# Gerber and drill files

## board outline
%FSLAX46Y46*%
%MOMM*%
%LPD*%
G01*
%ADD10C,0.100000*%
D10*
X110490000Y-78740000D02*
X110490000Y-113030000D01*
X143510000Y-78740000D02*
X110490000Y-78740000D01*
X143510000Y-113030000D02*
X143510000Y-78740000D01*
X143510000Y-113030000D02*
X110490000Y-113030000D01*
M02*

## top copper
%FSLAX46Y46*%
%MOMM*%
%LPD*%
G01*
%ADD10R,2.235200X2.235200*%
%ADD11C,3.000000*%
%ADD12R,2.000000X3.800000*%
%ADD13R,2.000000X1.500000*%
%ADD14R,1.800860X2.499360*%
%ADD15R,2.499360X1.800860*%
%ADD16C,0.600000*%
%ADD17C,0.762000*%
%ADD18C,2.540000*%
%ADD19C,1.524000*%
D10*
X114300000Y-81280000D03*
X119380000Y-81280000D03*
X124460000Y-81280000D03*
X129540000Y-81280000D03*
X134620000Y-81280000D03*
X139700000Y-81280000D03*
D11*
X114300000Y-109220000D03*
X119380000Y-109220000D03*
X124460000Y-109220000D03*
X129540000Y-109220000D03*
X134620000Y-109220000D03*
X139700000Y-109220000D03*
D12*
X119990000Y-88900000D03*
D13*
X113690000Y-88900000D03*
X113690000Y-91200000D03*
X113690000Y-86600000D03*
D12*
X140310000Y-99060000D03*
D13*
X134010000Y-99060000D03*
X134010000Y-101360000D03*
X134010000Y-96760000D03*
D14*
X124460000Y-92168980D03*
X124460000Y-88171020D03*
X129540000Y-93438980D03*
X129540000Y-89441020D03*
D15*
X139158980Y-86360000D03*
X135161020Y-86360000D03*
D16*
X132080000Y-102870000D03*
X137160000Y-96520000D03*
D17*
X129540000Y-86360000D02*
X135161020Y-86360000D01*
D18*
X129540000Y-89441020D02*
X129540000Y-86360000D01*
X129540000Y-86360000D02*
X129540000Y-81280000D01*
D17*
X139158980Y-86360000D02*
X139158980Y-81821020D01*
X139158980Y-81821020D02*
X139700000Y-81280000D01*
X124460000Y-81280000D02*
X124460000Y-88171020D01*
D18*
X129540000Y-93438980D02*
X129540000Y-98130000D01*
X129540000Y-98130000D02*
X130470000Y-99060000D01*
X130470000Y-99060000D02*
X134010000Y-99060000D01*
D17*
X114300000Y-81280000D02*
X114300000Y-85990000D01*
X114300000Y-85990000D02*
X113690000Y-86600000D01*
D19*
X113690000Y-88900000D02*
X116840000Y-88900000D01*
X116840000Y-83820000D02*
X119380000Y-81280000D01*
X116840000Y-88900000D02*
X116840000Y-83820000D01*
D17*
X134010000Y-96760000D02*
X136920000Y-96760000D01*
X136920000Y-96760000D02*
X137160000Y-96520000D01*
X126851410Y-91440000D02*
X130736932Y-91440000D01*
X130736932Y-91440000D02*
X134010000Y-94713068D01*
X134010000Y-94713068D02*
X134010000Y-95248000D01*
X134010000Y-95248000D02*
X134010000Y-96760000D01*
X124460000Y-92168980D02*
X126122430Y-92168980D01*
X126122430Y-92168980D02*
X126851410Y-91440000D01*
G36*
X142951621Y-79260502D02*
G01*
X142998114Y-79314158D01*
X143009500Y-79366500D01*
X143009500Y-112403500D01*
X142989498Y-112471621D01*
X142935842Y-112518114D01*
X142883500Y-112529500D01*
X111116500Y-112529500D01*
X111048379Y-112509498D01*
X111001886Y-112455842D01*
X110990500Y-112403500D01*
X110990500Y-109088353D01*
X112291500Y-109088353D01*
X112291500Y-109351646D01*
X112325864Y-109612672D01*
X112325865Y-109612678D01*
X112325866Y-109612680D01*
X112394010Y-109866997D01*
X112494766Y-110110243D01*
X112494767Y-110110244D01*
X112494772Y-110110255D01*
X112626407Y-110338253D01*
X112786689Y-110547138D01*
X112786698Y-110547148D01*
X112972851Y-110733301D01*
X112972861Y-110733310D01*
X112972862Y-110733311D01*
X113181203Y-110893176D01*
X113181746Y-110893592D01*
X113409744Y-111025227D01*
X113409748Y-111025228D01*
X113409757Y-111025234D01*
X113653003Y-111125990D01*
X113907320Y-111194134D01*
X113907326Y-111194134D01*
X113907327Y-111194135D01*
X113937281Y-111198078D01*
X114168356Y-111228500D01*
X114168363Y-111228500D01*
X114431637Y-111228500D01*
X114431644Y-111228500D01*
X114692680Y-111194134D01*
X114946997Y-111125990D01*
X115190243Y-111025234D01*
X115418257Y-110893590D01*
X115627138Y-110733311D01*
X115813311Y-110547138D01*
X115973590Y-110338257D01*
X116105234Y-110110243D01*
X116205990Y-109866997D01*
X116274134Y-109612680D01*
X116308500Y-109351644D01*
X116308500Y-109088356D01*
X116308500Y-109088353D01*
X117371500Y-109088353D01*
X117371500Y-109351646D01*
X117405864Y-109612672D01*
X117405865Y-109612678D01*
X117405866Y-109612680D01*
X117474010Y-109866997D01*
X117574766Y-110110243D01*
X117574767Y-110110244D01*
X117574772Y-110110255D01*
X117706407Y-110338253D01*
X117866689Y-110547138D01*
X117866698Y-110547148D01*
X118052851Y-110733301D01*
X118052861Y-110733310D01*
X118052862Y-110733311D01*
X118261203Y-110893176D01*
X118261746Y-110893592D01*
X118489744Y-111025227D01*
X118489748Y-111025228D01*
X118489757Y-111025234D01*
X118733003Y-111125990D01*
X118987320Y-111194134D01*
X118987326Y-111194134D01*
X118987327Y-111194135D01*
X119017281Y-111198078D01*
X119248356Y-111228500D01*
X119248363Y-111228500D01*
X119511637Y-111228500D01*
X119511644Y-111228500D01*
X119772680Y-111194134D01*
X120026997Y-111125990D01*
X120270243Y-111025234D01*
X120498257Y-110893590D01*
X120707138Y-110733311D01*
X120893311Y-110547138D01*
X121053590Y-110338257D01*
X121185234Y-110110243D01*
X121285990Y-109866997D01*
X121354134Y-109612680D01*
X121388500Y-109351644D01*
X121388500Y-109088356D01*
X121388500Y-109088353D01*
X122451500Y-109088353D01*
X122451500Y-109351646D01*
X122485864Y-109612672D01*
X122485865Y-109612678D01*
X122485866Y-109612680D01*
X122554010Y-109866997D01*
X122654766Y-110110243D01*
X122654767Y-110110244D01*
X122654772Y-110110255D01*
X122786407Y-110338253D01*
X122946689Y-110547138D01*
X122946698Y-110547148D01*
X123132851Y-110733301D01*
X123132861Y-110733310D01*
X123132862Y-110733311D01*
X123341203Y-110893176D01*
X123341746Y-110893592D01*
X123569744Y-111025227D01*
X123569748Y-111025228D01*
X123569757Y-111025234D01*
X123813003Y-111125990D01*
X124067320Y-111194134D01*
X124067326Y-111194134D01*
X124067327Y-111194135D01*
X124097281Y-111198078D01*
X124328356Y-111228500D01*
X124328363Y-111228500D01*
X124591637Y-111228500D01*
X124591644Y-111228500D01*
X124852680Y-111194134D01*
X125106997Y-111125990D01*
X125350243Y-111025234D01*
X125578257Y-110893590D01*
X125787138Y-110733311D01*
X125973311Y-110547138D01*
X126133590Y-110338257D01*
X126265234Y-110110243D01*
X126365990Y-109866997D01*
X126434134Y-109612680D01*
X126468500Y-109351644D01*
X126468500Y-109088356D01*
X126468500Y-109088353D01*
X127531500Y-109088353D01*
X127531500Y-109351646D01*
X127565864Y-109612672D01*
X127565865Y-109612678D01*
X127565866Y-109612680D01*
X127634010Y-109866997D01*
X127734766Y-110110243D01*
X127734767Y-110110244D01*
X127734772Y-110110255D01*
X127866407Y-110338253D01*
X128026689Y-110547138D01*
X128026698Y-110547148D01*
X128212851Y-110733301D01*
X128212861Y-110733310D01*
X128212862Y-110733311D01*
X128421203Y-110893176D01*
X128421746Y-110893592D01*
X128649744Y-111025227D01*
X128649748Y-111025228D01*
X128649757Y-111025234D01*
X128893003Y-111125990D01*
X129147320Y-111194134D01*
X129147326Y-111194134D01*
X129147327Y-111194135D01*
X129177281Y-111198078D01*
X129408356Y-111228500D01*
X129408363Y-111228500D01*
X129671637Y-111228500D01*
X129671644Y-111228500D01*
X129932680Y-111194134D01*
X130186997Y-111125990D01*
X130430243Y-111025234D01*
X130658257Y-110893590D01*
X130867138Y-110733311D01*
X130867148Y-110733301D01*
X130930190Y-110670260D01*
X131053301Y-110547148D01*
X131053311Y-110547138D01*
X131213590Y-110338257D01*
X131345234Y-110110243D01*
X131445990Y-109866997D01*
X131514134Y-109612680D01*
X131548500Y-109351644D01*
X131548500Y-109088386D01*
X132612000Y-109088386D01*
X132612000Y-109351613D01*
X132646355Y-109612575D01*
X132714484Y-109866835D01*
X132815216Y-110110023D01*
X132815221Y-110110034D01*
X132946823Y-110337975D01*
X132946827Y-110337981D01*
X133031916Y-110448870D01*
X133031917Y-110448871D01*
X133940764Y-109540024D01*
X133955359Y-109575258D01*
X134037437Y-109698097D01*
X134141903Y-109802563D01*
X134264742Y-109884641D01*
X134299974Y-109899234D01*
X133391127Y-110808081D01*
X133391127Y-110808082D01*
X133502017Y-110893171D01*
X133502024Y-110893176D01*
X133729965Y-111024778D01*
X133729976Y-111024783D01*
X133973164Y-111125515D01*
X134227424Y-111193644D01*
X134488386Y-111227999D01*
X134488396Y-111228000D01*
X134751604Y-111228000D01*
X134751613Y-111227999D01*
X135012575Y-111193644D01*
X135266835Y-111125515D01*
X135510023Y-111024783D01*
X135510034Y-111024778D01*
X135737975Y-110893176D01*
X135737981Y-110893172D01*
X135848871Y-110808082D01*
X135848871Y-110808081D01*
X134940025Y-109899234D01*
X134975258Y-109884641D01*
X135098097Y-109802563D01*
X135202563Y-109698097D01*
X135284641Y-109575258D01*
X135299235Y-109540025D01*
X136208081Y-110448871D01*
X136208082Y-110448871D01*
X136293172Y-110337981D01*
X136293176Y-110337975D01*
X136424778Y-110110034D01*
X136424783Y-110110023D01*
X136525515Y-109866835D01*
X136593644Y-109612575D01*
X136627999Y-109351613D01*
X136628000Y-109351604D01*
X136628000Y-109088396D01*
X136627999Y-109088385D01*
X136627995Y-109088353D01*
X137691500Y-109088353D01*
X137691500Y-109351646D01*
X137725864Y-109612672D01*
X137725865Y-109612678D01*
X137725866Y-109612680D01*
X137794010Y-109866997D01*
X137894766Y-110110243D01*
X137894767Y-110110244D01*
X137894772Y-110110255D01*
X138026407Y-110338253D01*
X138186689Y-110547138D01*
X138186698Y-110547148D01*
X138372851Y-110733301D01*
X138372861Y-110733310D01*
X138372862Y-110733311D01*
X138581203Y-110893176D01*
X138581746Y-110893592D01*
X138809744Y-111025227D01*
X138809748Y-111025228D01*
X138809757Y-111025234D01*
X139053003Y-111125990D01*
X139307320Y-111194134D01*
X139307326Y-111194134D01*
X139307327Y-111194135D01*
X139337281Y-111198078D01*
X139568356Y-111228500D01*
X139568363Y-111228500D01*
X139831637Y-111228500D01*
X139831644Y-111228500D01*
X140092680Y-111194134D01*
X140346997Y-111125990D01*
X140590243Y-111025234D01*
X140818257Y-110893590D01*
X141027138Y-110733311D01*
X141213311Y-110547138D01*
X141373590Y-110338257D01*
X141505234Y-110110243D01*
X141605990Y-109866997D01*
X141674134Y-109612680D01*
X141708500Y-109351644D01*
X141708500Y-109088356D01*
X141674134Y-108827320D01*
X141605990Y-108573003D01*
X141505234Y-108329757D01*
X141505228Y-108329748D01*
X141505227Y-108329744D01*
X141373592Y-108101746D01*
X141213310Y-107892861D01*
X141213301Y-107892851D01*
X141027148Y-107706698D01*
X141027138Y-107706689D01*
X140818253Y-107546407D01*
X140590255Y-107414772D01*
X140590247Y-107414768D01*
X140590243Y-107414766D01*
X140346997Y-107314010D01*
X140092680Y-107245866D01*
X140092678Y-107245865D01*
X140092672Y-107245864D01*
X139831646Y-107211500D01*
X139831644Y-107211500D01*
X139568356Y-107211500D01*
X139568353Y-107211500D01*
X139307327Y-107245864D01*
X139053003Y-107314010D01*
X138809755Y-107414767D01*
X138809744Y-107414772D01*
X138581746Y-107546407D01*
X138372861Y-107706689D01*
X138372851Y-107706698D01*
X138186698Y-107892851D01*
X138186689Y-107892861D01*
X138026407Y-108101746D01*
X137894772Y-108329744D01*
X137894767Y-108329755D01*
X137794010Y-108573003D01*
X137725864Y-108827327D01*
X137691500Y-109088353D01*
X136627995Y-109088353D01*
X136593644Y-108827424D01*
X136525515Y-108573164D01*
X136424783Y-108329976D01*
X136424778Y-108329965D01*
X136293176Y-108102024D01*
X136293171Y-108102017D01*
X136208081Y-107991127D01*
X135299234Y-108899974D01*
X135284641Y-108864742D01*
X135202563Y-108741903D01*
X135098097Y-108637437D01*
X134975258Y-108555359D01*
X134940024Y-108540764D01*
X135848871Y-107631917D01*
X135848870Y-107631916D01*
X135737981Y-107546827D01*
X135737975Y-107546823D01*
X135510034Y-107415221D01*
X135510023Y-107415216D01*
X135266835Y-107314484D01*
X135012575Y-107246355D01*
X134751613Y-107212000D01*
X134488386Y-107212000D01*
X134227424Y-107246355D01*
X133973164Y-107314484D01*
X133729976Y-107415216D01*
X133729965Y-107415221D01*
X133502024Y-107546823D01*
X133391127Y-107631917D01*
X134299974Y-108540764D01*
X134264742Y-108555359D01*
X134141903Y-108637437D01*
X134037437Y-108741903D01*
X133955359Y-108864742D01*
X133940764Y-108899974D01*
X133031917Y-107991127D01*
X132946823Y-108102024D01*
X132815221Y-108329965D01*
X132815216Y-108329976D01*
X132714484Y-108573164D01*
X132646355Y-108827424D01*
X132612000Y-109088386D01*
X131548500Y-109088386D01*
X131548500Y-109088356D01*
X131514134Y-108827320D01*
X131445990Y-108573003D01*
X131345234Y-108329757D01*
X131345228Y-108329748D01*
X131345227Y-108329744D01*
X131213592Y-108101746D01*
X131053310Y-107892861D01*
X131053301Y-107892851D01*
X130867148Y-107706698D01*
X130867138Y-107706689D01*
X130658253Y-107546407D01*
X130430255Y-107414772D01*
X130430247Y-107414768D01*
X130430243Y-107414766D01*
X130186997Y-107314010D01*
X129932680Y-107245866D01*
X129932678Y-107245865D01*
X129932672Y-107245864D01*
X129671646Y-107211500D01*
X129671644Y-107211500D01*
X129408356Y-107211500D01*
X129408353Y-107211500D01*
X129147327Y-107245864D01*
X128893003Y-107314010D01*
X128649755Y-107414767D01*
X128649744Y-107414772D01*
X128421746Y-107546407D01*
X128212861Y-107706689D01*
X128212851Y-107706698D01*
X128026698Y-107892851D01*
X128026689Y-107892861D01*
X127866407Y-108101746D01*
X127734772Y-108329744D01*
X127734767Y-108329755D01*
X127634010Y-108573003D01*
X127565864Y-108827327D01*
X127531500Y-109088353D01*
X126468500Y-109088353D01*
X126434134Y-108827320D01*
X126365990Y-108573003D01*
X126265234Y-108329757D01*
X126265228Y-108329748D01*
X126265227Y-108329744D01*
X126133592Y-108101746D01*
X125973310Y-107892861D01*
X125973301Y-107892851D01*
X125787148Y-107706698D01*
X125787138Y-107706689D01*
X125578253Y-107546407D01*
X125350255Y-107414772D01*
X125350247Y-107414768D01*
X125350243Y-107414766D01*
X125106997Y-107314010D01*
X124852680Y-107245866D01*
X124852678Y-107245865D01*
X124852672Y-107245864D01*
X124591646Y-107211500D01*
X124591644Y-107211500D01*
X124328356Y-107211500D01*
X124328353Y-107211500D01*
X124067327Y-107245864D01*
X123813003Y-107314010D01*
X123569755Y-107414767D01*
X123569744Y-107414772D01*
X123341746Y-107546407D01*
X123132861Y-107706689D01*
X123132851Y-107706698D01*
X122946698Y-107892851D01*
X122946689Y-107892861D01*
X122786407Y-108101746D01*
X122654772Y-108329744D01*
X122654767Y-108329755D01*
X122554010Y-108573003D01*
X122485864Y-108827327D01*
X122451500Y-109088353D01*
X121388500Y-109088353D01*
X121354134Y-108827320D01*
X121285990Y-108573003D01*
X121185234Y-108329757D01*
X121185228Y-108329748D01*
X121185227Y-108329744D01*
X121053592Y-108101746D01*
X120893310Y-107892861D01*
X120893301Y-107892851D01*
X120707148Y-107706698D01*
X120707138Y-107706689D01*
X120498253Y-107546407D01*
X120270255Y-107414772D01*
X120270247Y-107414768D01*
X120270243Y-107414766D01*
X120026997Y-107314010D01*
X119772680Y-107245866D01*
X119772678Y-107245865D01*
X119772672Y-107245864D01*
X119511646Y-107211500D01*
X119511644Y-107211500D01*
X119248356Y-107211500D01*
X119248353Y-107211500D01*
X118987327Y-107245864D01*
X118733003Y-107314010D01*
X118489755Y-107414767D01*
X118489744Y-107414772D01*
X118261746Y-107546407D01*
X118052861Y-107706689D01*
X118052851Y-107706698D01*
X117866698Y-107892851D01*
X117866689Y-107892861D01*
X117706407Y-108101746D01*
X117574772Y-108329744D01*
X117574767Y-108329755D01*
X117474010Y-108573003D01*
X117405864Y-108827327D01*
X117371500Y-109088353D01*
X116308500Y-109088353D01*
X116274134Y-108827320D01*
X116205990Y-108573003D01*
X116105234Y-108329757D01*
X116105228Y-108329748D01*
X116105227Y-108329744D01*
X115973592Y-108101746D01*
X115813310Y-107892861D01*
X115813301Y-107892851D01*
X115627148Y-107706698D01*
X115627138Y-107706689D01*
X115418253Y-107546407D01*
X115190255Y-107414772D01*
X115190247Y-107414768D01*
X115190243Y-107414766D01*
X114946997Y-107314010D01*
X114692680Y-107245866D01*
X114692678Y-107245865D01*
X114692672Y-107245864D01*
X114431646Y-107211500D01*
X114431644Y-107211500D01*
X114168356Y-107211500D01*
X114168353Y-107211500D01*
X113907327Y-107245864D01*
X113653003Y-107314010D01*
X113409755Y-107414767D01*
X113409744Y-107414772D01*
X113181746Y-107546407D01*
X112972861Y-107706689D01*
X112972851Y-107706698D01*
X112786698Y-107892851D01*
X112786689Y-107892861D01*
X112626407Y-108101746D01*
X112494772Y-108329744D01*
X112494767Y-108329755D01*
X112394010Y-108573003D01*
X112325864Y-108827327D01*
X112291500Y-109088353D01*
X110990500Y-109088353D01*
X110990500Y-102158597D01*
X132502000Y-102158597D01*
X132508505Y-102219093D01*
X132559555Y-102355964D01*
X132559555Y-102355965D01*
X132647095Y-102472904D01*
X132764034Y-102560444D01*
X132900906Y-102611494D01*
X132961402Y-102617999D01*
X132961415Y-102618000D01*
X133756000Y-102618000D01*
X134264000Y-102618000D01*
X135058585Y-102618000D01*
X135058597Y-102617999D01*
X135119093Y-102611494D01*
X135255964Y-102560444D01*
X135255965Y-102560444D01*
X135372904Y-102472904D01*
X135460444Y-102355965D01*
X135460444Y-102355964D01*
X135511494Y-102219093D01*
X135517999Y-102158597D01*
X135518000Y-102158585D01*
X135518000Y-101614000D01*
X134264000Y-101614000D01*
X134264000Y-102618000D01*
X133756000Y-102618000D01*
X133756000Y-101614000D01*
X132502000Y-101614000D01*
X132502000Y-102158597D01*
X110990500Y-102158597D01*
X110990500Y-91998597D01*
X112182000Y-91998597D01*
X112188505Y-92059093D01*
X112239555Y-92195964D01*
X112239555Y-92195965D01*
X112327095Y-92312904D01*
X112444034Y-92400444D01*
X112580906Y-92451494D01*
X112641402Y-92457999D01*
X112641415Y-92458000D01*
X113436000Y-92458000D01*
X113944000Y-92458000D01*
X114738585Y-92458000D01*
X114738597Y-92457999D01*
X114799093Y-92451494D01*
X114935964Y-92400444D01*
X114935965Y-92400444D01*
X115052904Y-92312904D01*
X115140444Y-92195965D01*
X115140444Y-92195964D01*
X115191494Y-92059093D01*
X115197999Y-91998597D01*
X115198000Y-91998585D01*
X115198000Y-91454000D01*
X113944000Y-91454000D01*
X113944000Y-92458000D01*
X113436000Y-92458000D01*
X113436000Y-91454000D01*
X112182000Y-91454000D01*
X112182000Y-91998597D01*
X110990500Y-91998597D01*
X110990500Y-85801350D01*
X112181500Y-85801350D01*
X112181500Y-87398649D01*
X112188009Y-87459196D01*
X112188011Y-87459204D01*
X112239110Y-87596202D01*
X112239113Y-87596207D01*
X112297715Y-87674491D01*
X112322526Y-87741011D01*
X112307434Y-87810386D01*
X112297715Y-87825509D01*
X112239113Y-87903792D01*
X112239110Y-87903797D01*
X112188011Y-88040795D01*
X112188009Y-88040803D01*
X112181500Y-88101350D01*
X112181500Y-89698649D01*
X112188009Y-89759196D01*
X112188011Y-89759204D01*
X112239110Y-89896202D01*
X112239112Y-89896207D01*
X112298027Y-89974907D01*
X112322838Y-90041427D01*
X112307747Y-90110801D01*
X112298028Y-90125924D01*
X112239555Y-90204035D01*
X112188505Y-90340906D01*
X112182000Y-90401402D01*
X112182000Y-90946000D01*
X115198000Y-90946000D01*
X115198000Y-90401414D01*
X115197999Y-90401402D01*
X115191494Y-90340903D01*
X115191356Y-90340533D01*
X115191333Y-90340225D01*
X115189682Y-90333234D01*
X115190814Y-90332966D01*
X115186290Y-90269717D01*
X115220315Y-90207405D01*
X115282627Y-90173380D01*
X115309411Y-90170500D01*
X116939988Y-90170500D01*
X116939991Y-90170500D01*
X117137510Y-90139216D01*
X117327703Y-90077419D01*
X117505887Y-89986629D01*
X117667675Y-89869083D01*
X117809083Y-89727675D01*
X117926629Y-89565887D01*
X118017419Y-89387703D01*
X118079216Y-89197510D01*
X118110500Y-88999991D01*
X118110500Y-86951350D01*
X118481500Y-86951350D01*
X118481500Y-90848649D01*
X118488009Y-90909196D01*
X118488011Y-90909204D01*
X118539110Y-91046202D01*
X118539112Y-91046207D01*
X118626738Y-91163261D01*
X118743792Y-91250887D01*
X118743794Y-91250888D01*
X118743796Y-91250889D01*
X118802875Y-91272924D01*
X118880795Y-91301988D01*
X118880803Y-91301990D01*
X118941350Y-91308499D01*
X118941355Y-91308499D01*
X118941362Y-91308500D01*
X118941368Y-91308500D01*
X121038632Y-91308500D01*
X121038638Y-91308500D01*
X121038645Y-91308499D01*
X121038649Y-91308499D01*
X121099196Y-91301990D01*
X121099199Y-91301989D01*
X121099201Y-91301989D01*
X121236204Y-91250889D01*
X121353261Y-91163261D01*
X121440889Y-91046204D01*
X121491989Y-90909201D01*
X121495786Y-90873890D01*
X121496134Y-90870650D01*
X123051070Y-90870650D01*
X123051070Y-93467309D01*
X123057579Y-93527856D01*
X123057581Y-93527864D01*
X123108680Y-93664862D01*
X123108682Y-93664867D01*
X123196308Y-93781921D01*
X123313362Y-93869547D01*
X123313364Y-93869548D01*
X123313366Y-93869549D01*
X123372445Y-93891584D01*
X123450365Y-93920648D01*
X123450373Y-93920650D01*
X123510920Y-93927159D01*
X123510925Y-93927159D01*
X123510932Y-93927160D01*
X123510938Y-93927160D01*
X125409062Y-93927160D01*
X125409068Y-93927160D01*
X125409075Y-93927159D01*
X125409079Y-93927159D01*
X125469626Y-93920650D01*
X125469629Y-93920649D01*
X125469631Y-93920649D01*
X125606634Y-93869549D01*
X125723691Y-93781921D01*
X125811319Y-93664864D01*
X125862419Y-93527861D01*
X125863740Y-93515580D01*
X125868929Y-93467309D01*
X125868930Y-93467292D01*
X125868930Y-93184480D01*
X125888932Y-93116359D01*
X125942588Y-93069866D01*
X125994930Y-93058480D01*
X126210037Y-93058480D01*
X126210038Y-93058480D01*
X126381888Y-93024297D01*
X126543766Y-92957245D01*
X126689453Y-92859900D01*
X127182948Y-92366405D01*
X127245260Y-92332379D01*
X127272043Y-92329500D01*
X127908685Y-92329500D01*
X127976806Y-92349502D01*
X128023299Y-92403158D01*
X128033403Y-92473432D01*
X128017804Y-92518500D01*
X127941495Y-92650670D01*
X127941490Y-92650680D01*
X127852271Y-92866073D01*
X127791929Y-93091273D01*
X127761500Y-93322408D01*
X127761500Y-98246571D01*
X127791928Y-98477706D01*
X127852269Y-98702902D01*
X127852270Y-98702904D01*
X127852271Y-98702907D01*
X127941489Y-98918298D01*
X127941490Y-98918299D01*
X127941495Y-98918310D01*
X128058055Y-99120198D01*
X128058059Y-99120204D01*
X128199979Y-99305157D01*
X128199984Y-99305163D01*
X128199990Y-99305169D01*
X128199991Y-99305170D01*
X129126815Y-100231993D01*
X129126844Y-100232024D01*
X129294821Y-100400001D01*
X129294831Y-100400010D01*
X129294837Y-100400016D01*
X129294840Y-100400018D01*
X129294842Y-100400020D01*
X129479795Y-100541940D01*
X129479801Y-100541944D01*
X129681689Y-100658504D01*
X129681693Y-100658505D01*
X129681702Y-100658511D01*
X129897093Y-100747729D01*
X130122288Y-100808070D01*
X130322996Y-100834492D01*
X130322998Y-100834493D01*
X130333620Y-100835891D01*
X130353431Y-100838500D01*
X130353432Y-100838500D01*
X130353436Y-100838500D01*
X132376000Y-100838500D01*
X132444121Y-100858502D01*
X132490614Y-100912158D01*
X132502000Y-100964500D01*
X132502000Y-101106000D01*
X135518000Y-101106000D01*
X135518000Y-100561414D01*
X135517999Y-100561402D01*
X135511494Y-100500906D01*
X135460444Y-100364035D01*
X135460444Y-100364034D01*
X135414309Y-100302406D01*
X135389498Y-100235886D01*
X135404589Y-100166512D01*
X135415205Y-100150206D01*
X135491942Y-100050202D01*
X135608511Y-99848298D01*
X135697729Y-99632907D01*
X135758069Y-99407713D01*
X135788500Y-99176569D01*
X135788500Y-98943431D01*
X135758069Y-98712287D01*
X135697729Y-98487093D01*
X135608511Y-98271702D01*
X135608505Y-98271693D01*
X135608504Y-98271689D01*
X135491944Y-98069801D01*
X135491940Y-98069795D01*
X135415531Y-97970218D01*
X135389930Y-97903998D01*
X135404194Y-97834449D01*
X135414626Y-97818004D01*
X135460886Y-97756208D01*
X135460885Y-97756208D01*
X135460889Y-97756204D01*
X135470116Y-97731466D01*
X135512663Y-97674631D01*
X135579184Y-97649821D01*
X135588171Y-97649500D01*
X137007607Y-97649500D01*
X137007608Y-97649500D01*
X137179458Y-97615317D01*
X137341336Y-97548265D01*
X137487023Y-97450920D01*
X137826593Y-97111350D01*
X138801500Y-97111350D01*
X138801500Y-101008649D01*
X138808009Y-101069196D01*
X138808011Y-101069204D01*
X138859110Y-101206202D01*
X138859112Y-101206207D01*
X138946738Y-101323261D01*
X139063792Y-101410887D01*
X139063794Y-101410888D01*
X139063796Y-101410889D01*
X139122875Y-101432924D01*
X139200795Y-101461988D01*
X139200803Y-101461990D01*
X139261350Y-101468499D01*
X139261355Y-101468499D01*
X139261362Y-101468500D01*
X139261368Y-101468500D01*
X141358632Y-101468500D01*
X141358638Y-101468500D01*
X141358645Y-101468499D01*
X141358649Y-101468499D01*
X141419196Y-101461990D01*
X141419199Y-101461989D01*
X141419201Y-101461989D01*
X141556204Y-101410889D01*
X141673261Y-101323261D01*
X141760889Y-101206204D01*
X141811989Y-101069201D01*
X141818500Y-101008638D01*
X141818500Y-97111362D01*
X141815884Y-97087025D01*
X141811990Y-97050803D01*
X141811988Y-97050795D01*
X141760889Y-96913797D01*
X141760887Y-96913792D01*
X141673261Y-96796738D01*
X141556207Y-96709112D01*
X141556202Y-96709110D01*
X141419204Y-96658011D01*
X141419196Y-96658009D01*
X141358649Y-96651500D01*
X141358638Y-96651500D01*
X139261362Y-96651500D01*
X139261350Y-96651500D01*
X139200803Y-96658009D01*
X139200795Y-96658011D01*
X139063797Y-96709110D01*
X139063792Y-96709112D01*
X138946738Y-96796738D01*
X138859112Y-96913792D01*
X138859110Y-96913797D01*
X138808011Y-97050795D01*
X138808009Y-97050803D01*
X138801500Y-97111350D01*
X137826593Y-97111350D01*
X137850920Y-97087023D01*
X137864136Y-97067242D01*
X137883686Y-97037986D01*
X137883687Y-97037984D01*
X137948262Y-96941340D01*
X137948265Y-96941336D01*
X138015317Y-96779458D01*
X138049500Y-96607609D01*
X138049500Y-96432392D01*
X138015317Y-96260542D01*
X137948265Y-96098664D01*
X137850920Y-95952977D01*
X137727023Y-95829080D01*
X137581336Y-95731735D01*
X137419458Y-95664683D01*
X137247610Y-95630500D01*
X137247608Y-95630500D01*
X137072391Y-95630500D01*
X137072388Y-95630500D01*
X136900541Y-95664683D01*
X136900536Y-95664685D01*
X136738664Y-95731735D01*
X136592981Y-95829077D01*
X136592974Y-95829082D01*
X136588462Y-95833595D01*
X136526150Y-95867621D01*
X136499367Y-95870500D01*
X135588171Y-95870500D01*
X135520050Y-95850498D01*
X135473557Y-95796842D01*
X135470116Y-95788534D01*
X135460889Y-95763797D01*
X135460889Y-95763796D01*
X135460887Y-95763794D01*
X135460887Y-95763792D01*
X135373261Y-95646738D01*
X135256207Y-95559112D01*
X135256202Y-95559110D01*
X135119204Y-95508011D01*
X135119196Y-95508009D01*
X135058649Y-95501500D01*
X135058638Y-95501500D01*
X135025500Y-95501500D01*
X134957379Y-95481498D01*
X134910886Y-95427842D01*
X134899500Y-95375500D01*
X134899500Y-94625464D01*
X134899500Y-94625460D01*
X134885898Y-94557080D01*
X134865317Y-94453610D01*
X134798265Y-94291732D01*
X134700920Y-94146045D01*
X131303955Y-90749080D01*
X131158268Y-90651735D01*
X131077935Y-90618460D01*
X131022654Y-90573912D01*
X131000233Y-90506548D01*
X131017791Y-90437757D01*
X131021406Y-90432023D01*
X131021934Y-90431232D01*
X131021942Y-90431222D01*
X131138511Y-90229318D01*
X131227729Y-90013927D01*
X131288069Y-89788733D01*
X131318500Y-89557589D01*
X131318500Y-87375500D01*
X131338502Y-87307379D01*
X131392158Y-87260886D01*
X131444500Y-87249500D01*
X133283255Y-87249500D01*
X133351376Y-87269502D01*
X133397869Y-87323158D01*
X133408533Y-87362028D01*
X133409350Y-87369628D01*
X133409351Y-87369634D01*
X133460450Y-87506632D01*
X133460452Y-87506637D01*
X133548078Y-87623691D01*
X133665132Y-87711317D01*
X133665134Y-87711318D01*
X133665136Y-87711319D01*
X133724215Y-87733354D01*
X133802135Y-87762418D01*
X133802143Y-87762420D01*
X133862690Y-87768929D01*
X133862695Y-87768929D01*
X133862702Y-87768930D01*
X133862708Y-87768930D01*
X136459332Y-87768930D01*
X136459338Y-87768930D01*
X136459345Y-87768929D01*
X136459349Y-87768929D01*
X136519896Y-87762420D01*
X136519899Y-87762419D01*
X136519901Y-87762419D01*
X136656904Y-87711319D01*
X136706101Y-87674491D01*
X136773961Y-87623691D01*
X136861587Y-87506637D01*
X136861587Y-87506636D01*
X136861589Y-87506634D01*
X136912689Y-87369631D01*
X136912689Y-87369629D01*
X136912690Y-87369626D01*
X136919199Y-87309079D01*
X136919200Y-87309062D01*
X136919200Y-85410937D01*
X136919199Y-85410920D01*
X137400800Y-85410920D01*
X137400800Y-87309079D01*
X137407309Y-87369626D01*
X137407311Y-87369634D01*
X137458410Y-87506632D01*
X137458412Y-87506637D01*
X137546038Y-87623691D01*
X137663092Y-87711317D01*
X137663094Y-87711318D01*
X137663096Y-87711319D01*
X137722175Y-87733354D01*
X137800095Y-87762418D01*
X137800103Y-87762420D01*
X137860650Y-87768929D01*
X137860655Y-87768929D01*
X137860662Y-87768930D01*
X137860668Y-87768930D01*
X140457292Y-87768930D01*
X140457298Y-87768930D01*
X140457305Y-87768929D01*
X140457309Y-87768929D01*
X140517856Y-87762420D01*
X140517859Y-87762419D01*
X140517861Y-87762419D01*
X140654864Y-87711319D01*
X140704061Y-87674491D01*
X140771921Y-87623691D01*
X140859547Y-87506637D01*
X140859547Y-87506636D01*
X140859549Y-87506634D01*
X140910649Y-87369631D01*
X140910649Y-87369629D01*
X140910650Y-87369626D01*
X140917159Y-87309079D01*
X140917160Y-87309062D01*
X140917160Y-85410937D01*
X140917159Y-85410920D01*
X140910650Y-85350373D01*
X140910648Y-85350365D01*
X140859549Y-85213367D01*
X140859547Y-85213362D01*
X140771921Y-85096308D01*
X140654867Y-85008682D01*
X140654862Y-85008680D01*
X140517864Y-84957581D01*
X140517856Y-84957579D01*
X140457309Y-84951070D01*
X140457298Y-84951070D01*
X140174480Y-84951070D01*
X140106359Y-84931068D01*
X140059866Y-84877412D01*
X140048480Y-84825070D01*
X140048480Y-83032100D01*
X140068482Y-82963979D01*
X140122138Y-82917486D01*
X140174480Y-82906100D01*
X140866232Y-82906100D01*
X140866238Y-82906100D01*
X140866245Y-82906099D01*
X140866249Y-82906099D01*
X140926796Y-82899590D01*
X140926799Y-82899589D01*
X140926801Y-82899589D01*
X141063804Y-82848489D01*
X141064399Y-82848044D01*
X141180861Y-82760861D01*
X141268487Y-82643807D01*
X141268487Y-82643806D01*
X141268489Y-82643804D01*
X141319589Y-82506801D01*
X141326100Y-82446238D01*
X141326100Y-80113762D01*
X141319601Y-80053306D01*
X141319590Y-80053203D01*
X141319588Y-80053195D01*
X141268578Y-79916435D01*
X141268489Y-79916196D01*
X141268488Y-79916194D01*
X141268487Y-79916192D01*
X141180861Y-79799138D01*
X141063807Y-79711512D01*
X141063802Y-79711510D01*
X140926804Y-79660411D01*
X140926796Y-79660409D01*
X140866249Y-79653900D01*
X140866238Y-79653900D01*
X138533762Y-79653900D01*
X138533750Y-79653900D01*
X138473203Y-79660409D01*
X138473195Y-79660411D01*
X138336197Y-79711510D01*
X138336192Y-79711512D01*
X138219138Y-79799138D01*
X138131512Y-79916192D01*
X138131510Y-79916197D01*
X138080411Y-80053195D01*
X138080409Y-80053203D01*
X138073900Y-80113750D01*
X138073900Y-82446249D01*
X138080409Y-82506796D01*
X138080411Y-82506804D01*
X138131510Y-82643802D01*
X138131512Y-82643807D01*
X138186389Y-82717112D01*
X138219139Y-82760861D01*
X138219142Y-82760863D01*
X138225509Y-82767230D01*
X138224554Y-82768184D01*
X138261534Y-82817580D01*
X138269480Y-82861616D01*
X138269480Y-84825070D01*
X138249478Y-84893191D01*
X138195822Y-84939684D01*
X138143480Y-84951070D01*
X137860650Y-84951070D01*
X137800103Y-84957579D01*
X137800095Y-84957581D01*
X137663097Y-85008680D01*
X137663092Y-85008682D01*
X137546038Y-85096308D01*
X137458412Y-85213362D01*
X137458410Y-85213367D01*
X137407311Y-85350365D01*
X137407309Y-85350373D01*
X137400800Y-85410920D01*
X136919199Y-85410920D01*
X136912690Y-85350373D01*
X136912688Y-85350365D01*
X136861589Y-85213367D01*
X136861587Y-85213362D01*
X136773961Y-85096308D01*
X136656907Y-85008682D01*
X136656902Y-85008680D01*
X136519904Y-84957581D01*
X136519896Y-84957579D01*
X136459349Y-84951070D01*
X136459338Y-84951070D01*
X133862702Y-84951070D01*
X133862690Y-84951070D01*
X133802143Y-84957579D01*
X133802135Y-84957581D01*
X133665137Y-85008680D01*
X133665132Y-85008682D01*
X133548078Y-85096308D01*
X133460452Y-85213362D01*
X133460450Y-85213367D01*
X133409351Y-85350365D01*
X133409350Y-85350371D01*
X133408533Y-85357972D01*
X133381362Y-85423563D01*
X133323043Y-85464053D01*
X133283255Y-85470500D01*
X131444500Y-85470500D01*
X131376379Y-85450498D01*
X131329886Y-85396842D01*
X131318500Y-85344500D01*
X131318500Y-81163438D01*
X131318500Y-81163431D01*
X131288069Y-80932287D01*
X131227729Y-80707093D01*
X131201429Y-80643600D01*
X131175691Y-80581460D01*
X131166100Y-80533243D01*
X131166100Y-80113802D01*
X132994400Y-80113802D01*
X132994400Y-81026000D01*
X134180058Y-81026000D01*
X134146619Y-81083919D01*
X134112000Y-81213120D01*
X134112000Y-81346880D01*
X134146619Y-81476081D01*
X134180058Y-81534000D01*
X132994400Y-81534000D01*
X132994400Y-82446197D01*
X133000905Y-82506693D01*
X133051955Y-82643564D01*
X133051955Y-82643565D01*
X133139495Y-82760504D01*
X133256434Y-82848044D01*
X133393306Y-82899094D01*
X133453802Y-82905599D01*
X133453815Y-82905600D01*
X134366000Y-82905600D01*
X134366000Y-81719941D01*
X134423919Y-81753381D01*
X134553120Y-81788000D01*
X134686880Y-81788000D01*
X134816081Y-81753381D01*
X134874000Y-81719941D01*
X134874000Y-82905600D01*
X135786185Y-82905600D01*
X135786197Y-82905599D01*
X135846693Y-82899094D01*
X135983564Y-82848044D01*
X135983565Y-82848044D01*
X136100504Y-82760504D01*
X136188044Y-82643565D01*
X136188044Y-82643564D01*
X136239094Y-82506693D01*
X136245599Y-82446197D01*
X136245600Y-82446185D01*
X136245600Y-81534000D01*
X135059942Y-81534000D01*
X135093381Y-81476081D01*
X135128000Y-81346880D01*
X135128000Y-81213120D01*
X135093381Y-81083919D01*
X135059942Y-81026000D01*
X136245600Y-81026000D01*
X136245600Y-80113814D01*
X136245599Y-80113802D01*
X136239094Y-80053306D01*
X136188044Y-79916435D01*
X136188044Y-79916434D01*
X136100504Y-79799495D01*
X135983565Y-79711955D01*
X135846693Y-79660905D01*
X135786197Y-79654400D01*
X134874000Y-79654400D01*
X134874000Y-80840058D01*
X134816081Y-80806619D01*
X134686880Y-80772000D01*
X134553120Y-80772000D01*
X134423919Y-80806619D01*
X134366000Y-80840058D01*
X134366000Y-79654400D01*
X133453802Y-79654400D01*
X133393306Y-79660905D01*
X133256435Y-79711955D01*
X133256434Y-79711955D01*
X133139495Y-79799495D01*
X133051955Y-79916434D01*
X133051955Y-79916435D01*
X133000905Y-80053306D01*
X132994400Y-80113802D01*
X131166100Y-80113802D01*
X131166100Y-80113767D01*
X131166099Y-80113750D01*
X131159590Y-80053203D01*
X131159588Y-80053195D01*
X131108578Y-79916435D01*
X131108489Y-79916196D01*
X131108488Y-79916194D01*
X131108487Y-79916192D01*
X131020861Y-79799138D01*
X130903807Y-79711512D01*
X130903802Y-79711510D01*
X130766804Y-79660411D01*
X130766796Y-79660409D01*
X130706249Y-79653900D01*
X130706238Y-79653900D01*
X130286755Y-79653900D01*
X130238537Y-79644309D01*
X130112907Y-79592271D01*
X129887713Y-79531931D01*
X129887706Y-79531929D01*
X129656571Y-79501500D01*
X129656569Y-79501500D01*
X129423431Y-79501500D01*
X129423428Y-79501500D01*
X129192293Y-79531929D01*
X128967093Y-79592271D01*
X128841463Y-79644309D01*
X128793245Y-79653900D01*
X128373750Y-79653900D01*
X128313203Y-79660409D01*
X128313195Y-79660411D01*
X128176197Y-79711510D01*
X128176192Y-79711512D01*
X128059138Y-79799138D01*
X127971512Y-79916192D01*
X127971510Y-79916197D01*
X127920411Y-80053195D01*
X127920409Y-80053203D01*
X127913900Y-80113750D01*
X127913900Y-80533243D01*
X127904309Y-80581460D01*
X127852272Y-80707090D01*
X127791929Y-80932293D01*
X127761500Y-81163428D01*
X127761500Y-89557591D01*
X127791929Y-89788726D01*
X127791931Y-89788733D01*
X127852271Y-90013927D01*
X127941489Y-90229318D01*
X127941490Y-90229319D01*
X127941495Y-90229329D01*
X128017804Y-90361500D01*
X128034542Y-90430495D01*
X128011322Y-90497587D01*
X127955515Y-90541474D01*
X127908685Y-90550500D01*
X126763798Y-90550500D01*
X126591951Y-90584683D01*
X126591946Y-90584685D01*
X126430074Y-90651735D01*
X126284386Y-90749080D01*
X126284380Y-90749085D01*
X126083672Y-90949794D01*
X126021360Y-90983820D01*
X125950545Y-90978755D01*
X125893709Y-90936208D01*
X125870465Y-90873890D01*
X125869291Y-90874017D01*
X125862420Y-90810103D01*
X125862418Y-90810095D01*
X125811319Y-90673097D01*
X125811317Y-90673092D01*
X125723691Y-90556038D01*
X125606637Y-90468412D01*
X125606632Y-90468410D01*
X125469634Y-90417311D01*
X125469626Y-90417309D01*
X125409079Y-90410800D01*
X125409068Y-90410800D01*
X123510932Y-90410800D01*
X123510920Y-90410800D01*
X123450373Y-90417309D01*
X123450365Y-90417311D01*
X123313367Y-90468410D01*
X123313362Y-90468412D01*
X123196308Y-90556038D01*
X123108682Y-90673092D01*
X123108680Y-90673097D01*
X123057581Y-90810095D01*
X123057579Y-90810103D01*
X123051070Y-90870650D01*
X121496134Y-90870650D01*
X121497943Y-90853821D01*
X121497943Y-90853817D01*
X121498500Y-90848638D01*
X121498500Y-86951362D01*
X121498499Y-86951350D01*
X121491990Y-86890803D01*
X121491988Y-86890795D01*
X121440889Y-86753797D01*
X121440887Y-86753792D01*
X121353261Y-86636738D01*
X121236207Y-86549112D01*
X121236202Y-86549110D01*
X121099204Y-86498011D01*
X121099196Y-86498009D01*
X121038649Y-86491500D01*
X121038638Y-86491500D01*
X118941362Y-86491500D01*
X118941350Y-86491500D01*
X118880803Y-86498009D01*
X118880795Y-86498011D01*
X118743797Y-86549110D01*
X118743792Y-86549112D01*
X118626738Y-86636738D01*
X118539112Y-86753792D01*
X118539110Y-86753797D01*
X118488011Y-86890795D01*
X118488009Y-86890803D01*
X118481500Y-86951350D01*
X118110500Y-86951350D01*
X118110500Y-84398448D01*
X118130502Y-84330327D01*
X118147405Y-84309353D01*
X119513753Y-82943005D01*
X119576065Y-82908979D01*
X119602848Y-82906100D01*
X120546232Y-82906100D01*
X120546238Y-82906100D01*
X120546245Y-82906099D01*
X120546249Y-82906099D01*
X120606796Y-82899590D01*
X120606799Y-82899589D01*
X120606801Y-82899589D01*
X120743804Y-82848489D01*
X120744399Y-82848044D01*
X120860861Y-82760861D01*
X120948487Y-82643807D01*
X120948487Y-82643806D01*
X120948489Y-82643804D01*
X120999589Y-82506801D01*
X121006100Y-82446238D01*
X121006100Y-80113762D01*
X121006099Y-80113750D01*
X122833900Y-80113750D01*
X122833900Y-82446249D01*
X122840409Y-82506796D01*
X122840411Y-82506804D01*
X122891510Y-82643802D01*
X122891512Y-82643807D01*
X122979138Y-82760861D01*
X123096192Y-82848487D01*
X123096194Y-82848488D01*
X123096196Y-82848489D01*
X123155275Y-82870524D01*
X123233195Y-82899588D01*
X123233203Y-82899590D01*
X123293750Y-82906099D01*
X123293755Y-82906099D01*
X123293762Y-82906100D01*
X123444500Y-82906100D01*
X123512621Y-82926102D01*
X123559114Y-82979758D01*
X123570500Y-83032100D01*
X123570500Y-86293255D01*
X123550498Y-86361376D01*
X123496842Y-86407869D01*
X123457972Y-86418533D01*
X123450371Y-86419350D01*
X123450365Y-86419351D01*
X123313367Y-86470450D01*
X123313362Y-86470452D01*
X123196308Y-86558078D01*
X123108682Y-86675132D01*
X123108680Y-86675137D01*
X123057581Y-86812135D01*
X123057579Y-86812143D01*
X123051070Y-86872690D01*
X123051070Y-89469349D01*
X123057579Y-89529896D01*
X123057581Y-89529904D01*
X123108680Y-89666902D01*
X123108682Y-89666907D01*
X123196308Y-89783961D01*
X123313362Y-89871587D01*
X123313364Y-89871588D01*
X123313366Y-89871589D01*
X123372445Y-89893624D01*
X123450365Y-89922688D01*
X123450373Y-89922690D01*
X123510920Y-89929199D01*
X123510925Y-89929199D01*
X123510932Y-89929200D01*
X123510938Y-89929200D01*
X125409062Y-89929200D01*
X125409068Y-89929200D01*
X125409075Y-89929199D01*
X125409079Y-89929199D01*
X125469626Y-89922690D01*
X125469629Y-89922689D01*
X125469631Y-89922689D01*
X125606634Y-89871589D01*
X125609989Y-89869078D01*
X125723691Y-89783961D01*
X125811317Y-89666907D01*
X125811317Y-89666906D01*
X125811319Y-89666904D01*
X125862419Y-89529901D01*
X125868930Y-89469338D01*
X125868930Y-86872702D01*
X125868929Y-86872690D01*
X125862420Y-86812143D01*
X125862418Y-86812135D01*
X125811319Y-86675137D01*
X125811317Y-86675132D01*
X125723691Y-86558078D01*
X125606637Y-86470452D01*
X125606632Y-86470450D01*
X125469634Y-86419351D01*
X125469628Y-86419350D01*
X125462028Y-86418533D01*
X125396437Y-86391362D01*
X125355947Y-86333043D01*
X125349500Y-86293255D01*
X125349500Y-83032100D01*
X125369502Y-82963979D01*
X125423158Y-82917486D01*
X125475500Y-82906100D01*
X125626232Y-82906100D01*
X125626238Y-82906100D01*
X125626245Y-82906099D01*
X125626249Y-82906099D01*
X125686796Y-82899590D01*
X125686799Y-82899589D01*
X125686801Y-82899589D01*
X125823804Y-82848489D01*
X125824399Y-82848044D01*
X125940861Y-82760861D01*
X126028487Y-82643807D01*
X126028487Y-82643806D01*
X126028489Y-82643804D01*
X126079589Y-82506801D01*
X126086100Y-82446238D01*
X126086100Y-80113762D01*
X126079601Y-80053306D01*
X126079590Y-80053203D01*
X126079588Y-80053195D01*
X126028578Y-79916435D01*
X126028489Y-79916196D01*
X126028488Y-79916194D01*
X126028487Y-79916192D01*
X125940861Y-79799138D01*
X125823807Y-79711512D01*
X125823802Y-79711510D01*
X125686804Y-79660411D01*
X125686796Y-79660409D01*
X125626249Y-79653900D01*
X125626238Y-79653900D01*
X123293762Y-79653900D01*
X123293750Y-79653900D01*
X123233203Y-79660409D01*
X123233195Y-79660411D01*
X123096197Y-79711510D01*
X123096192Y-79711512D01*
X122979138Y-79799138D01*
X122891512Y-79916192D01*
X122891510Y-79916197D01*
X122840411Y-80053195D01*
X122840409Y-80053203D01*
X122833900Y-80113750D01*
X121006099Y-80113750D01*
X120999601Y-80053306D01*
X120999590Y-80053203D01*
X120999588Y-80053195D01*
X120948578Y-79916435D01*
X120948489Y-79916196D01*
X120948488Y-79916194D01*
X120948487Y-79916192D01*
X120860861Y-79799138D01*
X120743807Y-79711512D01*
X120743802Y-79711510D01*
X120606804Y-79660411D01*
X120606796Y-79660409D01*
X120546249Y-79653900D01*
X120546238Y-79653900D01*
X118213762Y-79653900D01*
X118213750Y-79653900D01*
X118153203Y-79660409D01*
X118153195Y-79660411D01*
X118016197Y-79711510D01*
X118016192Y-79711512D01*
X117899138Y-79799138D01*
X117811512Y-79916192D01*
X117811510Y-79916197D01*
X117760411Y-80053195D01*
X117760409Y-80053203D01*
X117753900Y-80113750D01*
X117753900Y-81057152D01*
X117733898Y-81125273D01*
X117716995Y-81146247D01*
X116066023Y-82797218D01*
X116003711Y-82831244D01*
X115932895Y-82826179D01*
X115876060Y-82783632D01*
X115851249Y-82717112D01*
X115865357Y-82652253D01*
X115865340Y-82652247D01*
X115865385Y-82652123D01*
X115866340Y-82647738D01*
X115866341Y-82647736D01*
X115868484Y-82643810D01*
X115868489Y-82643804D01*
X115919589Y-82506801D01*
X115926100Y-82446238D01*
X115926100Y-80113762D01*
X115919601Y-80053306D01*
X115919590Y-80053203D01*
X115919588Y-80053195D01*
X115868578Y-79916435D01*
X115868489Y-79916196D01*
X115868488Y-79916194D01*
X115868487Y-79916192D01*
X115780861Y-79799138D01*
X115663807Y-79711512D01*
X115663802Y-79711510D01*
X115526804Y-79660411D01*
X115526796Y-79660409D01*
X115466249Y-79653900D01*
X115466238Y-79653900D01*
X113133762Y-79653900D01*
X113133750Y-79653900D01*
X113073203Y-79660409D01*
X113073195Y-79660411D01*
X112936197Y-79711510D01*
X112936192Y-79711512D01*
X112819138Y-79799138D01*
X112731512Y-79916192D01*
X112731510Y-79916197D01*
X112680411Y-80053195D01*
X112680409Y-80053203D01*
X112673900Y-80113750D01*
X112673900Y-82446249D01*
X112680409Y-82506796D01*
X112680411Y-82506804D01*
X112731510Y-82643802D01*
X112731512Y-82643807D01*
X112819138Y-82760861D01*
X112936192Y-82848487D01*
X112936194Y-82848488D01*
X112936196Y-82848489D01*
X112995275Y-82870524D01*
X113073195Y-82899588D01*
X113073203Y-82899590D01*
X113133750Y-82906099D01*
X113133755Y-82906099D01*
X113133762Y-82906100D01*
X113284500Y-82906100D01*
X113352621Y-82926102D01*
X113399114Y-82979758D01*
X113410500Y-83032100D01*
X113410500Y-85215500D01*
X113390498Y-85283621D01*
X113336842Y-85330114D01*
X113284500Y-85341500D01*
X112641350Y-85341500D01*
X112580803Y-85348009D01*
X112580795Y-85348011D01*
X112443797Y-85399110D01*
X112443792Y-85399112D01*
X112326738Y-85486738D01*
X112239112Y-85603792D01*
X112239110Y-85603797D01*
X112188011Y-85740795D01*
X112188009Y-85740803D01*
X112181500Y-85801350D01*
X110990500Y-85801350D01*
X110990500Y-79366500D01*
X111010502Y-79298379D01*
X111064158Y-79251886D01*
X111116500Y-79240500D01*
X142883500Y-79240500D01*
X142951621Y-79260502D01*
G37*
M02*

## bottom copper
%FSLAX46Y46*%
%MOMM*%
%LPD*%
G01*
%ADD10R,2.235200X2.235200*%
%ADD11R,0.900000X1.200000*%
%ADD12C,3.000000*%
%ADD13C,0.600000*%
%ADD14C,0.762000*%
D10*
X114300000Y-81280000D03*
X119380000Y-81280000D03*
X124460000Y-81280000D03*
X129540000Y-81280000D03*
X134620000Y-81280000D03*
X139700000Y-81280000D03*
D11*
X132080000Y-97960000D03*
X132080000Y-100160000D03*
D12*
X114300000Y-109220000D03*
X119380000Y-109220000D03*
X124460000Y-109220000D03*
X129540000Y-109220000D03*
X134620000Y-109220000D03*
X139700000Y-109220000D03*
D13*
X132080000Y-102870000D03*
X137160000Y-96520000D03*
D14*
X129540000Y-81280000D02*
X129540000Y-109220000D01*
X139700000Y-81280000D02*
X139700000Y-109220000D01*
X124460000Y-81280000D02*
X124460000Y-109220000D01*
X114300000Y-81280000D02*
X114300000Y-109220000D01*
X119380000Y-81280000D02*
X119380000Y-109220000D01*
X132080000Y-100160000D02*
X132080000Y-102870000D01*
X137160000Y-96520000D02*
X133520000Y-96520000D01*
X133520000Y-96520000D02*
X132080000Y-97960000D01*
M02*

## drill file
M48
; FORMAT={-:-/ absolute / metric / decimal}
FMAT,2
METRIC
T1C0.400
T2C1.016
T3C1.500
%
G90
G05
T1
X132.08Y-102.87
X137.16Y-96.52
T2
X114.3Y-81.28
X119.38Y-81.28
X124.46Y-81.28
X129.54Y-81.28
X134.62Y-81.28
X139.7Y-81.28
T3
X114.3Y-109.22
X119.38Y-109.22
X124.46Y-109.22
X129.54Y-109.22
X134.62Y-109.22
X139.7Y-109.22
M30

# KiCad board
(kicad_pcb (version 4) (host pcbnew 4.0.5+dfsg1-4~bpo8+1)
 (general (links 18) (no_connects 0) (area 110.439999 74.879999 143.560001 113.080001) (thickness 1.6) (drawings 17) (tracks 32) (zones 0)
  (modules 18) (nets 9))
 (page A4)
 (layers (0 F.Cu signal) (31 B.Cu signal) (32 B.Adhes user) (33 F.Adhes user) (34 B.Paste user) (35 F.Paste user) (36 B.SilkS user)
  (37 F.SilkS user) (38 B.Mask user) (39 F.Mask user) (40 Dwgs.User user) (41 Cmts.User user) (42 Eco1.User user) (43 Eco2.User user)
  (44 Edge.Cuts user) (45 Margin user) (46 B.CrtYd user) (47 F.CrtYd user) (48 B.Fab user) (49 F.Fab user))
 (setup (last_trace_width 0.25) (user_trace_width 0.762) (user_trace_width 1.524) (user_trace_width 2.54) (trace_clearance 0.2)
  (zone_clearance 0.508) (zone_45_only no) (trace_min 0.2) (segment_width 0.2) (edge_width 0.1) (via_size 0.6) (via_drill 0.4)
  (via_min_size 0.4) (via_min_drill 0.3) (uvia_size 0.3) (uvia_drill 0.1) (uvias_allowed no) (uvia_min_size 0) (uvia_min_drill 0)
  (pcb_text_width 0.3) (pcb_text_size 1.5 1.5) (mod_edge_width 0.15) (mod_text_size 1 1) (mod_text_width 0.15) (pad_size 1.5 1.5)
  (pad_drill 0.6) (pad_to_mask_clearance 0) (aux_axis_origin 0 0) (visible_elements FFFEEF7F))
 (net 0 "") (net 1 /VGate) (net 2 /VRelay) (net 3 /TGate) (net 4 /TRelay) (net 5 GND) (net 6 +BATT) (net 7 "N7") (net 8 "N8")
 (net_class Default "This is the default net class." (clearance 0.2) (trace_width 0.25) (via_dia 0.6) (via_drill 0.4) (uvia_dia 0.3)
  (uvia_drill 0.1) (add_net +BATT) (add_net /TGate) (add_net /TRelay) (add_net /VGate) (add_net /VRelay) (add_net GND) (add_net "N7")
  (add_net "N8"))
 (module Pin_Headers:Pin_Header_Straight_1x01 (layer B.Cu) (at 114.3 81.28)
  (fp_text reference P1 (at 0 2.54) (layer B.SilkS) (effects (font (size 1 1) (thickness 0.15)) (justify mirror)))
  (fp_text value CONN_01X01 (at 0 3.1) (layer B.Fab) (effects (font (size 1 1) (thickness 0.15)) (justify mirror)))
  (pad 1 thru_hole rect (at 0 0) (size 2.2352 2.2352) (drill 1.016) (layers *.Cu *.Mask) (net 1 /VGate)))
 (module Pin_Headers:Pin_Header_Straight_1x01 (layer B.Cu) (at 119.38 81.28)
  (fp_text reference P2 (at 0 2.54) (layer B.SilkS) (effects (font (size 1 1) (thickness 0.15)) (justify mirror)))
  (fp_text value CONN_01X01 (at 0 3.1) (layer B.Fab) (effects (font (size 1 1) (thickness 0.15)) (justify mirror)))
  (pad 1 thru_hole rect (at 0 0) (size 2.2352 2.2352) (drill 1.016) (layers *.Cu *.Mask) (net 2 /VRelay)))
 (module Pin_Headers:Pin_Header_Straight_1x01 (layer B.Cu) (at 124.46 81.28)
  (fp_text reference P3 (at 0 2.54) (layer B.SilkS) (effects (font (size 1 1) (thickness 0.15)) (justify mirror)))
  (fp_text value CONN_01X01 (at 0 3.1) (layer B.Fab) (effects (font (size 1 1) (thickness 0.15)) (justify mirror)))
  (pad 1 thru_hole rect (at 0 0) (size 2.2352 2.2352) (drill 1.016) (layers *.Cu *.Mask) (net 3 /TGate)))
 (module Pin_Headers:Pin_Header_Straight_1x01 (layer B.Cu) (at 129.54 81.28)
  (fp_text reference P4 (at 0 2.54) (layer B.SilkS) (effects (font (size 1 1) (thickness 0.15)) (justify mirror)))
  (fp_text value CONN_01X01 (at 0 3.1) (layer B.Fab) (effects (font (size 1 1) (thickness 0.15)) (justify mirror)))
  (pad 1 thru_hole rect (at 0 0) (size 2.2352 2.2352) (drill 1.016) (layers *.Cu *.Mask) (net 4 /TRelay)))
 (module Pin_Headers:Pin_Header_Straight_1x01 (layer B.Cu) (at 134.62 81.28)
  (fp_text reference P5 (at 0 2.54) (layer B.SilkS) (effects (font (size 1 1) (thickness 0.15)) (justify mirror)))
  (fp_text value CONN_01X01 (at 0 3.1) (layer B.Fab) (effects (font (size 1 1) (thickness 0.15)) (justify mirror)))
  (pad 1 thru_hole rect (at 0 0) (size 2.2352 2.2352) (drill 1.016) (layers *.Cu *.Mask) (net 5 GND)))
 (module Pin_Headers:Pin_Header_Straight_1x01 (layer B.Cu) (at 139.7 81.28)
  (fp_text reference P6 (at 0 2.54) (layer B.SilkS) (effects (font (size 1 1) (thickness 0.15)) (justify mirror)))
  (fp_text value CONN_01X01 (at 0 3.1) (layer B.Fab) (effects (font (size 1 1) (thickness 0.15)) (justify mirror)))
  (pad 1 thru_hole rect (at 0 0) (size 2.2352 2.2352) (drill 1.016) (layers *.Cu *.Mask) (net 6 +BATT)))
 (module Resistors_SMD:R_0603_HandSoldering (layer B.Cu) (at 132.08 99.06 270)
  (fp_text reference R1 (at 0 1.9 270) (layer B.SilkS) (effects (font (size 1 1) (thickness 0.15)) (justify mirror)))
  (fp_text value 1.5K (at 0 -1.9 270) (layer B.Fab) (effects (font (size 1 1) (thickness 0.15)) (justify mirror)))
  (pad 1 smd rect (at -1.1 0 270) (size 1.2 0.9) (layers B.Cu B.Paste B.Mask) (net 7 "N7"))
  (pad 2 smd rect (at 1.1 0 270) (size 1.2 0.9) (layers B.Cu B.Paste B.Mask) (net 5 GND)))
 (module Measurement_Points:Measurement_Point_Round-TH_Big (layer B.Cu) (at 114.3 109.22)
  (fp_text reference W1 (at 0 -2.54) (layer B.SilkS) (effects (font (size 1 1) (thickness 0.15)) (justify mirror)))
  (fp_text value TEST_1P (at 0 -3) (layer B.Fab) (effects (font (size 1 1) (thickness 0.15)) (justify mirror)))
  (pad 1 thru_hole circle (at 0 0) (size 3 3) (drill 1.5) (layers *.Cu *.Mask) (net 1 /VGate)))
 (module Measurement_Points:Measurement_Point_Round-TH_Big (layer B.Cu) (at 119.38 109.22)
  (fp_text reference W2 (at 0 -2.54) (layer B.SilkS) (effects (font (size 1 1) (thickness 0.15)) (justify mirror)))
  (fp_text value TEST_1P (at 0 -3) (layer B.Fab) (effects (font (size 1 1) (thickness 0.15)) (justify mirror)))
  (pad 1 thru_hole circle (at 0 0) (size 3 3) (drill 1.5) (layers *.Cu *.Mask) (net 2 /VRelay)))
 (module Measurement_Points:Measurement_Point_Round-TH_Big (layer B.Cu) (at 124.46 109.22)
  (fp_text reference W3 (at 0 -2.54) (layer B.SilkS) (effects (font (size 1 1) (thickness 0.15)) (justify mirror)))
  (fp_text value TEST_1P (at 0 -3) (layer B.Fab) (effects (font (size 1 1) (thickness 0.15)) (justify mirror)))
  (pad 1 thru_hole circle (at 0 0) (size 3 3) (drill 1.5) (layers *.Cu *.Mask) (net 3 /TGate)))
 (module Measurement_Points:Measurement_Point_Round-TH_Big (layer B.Cu) (at 129.54 109.22)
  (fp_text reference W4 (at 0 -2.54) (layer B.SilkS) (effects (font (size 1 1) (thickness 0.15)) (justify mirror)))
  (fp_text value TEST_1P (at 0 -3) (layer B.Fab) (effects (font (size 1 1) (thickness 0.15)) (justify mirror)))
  (pad 1 thru_hole circle (at 0 0) (size 3 3) (drill 1.5) (layers *.Cu *.Mask) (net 4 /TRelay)))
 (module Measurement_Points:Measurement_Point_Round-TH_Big (layer B.Cu) (at 134.62 109.22)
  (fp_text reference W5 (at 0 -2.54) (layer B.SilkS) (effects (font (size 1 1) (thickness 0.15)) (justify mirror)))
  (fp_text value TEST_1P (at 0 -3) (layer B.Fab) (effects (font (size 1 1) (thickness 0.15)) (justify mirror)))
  (pad 1 thru_hole circle (at 0 0) (size 3 3) (drill 1.5) (layers *.Cu *.Mask) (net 5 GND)))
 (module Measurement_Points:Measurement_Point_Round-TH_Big (layer B.Cu) (at 139.7 109.22)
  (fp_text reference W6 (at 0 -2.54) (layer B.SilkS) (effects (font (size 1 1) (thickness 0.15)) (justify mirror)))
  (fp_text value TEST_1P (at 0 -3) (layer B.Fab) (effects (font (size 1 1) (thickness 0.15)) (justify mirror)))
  (pad 1 thru_hole circle (at 0 0) (size 3 3) (drill 1.5) (layers *.Cu *.Mask) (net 6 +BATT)))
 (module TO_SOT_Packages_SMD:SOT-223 (layer F.Cu) (at 116.84 88.9)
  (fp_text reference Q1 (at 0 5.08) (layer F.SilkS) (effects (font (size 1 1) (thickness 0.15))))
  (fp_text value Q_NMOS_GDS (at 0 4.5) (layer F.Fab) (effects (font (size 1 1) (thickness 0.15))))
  (pad 4 smd rect (at 3.15 0) (size 2 3.8) (layers F.Cu F.Paste F.Mask))
  (pad 2 smd rect (at -3.15 0) (size 2 1.5) (layers F.Cu F.Paste F.Mask) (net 2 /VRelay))
  (pad 3 smd rect (at -3.15 2.3) (size 2 1.5) (layers F.Cu F.Paste F.Mask) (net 5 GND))
  (pad 1 smd rect (at -3.15 -2.3) (size 2 1.5) (layers F.Cu F.Paste F.Mask) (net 1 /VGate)))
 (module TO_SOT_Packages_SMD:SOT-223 (layer F.Cu) (at 137.16 99.06)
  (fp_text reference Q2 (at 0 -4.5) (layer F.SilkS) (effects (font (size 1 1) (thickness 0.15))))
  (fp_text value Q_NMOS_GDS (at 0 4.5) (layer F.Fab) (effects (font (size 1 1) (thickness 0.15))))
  (pad 4 smd rect (at 3.15 0) (size 2 3.8) (layers F.Cu F.Paste F.Mask))
  (pad 2 smd rect (at -3.15 0) (size 2 1.5) (layers F.Cu F.Paste F.Mask) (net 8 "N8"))
  (pad 3 smd rect (at -3.15 2.3) (size 2 1.5) (layers F.Cu F.Paste F.Mask) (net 5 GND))
  (pad 1 smd rect (at -3.15 -2.3) (size 2 1.5) (layers F.Cu F.Paste F.Mask) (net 7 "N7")))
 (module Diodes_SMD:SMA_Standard (layer F.Cu) (at 124.46 90.17 90)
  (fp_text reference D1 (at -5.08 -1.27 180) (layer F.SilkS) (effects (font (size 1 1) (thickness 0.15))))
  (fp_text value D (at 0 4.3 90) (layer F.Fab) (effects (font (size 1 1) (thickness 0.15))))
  (pad 1 smd rect (at -1.99898 0 90) (size 2.49936 1.80086) (layers F.Cu F.Paste F.Mask) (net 7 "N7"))
  (pad 2 smd rect (at 1.99898 0 90) (size 2.49936 1.80086) (layers F.Cu F.Paste F.Mask) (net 3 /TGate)))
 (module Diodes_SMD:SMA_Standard (layer F.Cu) (at 129.54 91.44 90)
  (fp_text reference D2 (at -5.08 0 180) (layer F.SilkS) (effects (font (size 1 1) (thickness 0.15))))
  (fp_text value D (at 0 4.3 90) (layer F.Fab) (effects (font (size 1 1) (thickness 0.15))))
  (pad 1 smd rect (at -1.99898 0 90) (size 2.49936 1.80086) (layers F.Cu F.Paste F.Mask) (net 8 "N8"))
  (pad 2 smd rect (at 1.99898 0 90) (size 2.49936 1.80086) (layers F.Cu F.Paste F.Mask) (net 4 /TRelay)))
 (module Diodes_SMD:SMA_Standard (layer F.Cu) (at 137.16 86.36 180)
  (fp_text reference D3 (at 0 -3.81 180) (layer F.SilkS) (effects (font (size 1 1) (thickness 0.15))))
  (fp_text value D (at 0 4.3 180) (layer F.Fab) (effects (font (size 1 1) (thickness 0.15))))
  (pad 1 smd rect (at -1.99898 0 180) (size 2.49936 1.80086) (layers F.Cu F.Paste F.Mask) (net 6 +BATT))
  (pad 2 smd rect (at 1.99898 0 180) (size 2.49936 1.80086) (layers F.Cu F.Paste F.Mask) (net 4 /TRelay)))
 (gr_line (start 110.49 78.74) (end 110.49 113.03) (angle 90) (layer Edge.Cuts) (width 0.1))
 (gr_line (start 143.51 78.74) (end 110.49 78.74) (angle 90) (layer Edge.Cuts) (width 0.1))
 (gr_line (start 143.51 113.03) (end 143.51 78.74) (angle 90) (layer Edge.Cuts) (width 0.1))
 (gr_line (start 143.51 113.03) (end 110.49 113.03) (angle 90) (layer Edge.Cuts) (width 0.1))
 (segment (start 129.54 86.36) (end 135.16102 86.36) (width 0.762) (layer F.Cu) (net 4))
 (segment (start 129.54 89.44102) (end 129.54 86.36) (width 2.54) (layer F.Cu) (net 4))
 (segment (start 129.54 86.36) (end 129.54 81.28) (width 2.54) (layer F.Cu) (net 4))
 (segment (start 129.54 81.28) (end 129.54 109.22) (width 0.762) (layer B.Cu) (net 4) (status 30))
 (segment (start 139.15898 86.36) (end 139.15898 81.82102) (width 0.762) (layer F.Cu) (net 6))
 (segment (start 139.15898 81.82102) (end 139.7 81.28) (width 0.762) (layer F.Cu) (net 6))
 (segment (start 139.7 81.28) (end 139.7 109.22) (width 0.762) (layer B.Cu) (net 6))
 (segment (start 124.46 81.28) (end 124.46 88.17102) (width 0.762) (layer F.Cu) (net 3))
 (segment (start 124.46 81.28) (end 124.46 109.22) (width 0.762) (layer B.Cu) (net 3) (status 30))
 (segment (start 129.54 93.43898) (end 129.54 98.13) (width 2.54) (layer F.Cu) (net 8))
 (segment (start 129.54 98.13) (end 130.47 99.06) (width 2.54) (layer F.Cu) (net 8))
 (segment (start 130.47 99.06) (end 134.01 99.06) (width 2.54) (layer F.Cu) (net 8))
 (segment (start 114.3 81.28) (end 114.3 109.22) (width 0.762) (layer B.Cu) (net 1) (status 30))
 (segment (start 114.3 81.28) (end 114.3 85.99) (width 0.762) (layer F.Cu) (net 1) (status 30))
 (segment (start 114.3 85.99) (end 113.69 86.6) (width 0.762) (layer F.Cu) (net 1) (status 30))
 (segment (start 113.69 88.9) (end 116.84 88.9) (width 1.524) (layer F.Cu) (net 2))
 (segment (start 116.84 83.82) (end 119.38 81.28) (width 1.524) (layer F.Cu) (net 2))
 (segment (start 116.84 88.9) (end 116.84 83.82) (width 1.524) (layer F.Cu) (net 2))
 (segment (start 119.38 81.28) (end 119.38 109.22) (width 0.762) (layer B.Cu) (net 2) (status 30))
 (segment (start 132.08 100.16) (end 132.08 102.87) (width 0.762) (layer B.Cu) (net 5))
 (via (at 132.08 102.87) (size 0.6) (drill 0.4) (layers F.Cu B.Cu) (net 5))
 (segment (start 137.16 96.52) (end 133.52 96.52) (width 0.762) (layer B.Cu) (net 7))
 (segment (start 133.52 96.52) (end 132.08 97.96) (width 0.762) (layer B.Cu) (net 7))
 (segment (start 134.01 96.76) (end 136.92 96.76) (width 0.762) (layer F.Cu) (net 7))
 (segment (start 136.92 96.76) (end 137.16 96.52) (width 0.762) (layer F.Cu) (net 7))
 (via (at 137.16 96.52) (size 0.6) (drill 0.4) (layers F.Cu B.Cu) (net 7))
 (segment (start 126.85141 91.44) (end 130.736932 91.44) (width 0.762) (layer F.Cu) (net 7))
 (segment (start 130.736932 91.44) (end 134.01 94.713068) (width 0.762) (layer F.Cu) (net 7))
 (segment (start 134.01 94.713068) (end 134.01 95.248) (width 0.762) (layer F.Cu) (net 7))
 (segment (start 134.01 95.248) (end 134.01 96.76) (width 0.762) (layer F.Cu) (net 7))
 (segment (start 124.46 92.16898) (end 126.12243 92.16898) (width 0.762) (layer F.Cu) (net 7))
 (segment (start 126.12243 92.16898) (end 126.85141 91.44) (width 0.762) (layer F.Cu) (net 7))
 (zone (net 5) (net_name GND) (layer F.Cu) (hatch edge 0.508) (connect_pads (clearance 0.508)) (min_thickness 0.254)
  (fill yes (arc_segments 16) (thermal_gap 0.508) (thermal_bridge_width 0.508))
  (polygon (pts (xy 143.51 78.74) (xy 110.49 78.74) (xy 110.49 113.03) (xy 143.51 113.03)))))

